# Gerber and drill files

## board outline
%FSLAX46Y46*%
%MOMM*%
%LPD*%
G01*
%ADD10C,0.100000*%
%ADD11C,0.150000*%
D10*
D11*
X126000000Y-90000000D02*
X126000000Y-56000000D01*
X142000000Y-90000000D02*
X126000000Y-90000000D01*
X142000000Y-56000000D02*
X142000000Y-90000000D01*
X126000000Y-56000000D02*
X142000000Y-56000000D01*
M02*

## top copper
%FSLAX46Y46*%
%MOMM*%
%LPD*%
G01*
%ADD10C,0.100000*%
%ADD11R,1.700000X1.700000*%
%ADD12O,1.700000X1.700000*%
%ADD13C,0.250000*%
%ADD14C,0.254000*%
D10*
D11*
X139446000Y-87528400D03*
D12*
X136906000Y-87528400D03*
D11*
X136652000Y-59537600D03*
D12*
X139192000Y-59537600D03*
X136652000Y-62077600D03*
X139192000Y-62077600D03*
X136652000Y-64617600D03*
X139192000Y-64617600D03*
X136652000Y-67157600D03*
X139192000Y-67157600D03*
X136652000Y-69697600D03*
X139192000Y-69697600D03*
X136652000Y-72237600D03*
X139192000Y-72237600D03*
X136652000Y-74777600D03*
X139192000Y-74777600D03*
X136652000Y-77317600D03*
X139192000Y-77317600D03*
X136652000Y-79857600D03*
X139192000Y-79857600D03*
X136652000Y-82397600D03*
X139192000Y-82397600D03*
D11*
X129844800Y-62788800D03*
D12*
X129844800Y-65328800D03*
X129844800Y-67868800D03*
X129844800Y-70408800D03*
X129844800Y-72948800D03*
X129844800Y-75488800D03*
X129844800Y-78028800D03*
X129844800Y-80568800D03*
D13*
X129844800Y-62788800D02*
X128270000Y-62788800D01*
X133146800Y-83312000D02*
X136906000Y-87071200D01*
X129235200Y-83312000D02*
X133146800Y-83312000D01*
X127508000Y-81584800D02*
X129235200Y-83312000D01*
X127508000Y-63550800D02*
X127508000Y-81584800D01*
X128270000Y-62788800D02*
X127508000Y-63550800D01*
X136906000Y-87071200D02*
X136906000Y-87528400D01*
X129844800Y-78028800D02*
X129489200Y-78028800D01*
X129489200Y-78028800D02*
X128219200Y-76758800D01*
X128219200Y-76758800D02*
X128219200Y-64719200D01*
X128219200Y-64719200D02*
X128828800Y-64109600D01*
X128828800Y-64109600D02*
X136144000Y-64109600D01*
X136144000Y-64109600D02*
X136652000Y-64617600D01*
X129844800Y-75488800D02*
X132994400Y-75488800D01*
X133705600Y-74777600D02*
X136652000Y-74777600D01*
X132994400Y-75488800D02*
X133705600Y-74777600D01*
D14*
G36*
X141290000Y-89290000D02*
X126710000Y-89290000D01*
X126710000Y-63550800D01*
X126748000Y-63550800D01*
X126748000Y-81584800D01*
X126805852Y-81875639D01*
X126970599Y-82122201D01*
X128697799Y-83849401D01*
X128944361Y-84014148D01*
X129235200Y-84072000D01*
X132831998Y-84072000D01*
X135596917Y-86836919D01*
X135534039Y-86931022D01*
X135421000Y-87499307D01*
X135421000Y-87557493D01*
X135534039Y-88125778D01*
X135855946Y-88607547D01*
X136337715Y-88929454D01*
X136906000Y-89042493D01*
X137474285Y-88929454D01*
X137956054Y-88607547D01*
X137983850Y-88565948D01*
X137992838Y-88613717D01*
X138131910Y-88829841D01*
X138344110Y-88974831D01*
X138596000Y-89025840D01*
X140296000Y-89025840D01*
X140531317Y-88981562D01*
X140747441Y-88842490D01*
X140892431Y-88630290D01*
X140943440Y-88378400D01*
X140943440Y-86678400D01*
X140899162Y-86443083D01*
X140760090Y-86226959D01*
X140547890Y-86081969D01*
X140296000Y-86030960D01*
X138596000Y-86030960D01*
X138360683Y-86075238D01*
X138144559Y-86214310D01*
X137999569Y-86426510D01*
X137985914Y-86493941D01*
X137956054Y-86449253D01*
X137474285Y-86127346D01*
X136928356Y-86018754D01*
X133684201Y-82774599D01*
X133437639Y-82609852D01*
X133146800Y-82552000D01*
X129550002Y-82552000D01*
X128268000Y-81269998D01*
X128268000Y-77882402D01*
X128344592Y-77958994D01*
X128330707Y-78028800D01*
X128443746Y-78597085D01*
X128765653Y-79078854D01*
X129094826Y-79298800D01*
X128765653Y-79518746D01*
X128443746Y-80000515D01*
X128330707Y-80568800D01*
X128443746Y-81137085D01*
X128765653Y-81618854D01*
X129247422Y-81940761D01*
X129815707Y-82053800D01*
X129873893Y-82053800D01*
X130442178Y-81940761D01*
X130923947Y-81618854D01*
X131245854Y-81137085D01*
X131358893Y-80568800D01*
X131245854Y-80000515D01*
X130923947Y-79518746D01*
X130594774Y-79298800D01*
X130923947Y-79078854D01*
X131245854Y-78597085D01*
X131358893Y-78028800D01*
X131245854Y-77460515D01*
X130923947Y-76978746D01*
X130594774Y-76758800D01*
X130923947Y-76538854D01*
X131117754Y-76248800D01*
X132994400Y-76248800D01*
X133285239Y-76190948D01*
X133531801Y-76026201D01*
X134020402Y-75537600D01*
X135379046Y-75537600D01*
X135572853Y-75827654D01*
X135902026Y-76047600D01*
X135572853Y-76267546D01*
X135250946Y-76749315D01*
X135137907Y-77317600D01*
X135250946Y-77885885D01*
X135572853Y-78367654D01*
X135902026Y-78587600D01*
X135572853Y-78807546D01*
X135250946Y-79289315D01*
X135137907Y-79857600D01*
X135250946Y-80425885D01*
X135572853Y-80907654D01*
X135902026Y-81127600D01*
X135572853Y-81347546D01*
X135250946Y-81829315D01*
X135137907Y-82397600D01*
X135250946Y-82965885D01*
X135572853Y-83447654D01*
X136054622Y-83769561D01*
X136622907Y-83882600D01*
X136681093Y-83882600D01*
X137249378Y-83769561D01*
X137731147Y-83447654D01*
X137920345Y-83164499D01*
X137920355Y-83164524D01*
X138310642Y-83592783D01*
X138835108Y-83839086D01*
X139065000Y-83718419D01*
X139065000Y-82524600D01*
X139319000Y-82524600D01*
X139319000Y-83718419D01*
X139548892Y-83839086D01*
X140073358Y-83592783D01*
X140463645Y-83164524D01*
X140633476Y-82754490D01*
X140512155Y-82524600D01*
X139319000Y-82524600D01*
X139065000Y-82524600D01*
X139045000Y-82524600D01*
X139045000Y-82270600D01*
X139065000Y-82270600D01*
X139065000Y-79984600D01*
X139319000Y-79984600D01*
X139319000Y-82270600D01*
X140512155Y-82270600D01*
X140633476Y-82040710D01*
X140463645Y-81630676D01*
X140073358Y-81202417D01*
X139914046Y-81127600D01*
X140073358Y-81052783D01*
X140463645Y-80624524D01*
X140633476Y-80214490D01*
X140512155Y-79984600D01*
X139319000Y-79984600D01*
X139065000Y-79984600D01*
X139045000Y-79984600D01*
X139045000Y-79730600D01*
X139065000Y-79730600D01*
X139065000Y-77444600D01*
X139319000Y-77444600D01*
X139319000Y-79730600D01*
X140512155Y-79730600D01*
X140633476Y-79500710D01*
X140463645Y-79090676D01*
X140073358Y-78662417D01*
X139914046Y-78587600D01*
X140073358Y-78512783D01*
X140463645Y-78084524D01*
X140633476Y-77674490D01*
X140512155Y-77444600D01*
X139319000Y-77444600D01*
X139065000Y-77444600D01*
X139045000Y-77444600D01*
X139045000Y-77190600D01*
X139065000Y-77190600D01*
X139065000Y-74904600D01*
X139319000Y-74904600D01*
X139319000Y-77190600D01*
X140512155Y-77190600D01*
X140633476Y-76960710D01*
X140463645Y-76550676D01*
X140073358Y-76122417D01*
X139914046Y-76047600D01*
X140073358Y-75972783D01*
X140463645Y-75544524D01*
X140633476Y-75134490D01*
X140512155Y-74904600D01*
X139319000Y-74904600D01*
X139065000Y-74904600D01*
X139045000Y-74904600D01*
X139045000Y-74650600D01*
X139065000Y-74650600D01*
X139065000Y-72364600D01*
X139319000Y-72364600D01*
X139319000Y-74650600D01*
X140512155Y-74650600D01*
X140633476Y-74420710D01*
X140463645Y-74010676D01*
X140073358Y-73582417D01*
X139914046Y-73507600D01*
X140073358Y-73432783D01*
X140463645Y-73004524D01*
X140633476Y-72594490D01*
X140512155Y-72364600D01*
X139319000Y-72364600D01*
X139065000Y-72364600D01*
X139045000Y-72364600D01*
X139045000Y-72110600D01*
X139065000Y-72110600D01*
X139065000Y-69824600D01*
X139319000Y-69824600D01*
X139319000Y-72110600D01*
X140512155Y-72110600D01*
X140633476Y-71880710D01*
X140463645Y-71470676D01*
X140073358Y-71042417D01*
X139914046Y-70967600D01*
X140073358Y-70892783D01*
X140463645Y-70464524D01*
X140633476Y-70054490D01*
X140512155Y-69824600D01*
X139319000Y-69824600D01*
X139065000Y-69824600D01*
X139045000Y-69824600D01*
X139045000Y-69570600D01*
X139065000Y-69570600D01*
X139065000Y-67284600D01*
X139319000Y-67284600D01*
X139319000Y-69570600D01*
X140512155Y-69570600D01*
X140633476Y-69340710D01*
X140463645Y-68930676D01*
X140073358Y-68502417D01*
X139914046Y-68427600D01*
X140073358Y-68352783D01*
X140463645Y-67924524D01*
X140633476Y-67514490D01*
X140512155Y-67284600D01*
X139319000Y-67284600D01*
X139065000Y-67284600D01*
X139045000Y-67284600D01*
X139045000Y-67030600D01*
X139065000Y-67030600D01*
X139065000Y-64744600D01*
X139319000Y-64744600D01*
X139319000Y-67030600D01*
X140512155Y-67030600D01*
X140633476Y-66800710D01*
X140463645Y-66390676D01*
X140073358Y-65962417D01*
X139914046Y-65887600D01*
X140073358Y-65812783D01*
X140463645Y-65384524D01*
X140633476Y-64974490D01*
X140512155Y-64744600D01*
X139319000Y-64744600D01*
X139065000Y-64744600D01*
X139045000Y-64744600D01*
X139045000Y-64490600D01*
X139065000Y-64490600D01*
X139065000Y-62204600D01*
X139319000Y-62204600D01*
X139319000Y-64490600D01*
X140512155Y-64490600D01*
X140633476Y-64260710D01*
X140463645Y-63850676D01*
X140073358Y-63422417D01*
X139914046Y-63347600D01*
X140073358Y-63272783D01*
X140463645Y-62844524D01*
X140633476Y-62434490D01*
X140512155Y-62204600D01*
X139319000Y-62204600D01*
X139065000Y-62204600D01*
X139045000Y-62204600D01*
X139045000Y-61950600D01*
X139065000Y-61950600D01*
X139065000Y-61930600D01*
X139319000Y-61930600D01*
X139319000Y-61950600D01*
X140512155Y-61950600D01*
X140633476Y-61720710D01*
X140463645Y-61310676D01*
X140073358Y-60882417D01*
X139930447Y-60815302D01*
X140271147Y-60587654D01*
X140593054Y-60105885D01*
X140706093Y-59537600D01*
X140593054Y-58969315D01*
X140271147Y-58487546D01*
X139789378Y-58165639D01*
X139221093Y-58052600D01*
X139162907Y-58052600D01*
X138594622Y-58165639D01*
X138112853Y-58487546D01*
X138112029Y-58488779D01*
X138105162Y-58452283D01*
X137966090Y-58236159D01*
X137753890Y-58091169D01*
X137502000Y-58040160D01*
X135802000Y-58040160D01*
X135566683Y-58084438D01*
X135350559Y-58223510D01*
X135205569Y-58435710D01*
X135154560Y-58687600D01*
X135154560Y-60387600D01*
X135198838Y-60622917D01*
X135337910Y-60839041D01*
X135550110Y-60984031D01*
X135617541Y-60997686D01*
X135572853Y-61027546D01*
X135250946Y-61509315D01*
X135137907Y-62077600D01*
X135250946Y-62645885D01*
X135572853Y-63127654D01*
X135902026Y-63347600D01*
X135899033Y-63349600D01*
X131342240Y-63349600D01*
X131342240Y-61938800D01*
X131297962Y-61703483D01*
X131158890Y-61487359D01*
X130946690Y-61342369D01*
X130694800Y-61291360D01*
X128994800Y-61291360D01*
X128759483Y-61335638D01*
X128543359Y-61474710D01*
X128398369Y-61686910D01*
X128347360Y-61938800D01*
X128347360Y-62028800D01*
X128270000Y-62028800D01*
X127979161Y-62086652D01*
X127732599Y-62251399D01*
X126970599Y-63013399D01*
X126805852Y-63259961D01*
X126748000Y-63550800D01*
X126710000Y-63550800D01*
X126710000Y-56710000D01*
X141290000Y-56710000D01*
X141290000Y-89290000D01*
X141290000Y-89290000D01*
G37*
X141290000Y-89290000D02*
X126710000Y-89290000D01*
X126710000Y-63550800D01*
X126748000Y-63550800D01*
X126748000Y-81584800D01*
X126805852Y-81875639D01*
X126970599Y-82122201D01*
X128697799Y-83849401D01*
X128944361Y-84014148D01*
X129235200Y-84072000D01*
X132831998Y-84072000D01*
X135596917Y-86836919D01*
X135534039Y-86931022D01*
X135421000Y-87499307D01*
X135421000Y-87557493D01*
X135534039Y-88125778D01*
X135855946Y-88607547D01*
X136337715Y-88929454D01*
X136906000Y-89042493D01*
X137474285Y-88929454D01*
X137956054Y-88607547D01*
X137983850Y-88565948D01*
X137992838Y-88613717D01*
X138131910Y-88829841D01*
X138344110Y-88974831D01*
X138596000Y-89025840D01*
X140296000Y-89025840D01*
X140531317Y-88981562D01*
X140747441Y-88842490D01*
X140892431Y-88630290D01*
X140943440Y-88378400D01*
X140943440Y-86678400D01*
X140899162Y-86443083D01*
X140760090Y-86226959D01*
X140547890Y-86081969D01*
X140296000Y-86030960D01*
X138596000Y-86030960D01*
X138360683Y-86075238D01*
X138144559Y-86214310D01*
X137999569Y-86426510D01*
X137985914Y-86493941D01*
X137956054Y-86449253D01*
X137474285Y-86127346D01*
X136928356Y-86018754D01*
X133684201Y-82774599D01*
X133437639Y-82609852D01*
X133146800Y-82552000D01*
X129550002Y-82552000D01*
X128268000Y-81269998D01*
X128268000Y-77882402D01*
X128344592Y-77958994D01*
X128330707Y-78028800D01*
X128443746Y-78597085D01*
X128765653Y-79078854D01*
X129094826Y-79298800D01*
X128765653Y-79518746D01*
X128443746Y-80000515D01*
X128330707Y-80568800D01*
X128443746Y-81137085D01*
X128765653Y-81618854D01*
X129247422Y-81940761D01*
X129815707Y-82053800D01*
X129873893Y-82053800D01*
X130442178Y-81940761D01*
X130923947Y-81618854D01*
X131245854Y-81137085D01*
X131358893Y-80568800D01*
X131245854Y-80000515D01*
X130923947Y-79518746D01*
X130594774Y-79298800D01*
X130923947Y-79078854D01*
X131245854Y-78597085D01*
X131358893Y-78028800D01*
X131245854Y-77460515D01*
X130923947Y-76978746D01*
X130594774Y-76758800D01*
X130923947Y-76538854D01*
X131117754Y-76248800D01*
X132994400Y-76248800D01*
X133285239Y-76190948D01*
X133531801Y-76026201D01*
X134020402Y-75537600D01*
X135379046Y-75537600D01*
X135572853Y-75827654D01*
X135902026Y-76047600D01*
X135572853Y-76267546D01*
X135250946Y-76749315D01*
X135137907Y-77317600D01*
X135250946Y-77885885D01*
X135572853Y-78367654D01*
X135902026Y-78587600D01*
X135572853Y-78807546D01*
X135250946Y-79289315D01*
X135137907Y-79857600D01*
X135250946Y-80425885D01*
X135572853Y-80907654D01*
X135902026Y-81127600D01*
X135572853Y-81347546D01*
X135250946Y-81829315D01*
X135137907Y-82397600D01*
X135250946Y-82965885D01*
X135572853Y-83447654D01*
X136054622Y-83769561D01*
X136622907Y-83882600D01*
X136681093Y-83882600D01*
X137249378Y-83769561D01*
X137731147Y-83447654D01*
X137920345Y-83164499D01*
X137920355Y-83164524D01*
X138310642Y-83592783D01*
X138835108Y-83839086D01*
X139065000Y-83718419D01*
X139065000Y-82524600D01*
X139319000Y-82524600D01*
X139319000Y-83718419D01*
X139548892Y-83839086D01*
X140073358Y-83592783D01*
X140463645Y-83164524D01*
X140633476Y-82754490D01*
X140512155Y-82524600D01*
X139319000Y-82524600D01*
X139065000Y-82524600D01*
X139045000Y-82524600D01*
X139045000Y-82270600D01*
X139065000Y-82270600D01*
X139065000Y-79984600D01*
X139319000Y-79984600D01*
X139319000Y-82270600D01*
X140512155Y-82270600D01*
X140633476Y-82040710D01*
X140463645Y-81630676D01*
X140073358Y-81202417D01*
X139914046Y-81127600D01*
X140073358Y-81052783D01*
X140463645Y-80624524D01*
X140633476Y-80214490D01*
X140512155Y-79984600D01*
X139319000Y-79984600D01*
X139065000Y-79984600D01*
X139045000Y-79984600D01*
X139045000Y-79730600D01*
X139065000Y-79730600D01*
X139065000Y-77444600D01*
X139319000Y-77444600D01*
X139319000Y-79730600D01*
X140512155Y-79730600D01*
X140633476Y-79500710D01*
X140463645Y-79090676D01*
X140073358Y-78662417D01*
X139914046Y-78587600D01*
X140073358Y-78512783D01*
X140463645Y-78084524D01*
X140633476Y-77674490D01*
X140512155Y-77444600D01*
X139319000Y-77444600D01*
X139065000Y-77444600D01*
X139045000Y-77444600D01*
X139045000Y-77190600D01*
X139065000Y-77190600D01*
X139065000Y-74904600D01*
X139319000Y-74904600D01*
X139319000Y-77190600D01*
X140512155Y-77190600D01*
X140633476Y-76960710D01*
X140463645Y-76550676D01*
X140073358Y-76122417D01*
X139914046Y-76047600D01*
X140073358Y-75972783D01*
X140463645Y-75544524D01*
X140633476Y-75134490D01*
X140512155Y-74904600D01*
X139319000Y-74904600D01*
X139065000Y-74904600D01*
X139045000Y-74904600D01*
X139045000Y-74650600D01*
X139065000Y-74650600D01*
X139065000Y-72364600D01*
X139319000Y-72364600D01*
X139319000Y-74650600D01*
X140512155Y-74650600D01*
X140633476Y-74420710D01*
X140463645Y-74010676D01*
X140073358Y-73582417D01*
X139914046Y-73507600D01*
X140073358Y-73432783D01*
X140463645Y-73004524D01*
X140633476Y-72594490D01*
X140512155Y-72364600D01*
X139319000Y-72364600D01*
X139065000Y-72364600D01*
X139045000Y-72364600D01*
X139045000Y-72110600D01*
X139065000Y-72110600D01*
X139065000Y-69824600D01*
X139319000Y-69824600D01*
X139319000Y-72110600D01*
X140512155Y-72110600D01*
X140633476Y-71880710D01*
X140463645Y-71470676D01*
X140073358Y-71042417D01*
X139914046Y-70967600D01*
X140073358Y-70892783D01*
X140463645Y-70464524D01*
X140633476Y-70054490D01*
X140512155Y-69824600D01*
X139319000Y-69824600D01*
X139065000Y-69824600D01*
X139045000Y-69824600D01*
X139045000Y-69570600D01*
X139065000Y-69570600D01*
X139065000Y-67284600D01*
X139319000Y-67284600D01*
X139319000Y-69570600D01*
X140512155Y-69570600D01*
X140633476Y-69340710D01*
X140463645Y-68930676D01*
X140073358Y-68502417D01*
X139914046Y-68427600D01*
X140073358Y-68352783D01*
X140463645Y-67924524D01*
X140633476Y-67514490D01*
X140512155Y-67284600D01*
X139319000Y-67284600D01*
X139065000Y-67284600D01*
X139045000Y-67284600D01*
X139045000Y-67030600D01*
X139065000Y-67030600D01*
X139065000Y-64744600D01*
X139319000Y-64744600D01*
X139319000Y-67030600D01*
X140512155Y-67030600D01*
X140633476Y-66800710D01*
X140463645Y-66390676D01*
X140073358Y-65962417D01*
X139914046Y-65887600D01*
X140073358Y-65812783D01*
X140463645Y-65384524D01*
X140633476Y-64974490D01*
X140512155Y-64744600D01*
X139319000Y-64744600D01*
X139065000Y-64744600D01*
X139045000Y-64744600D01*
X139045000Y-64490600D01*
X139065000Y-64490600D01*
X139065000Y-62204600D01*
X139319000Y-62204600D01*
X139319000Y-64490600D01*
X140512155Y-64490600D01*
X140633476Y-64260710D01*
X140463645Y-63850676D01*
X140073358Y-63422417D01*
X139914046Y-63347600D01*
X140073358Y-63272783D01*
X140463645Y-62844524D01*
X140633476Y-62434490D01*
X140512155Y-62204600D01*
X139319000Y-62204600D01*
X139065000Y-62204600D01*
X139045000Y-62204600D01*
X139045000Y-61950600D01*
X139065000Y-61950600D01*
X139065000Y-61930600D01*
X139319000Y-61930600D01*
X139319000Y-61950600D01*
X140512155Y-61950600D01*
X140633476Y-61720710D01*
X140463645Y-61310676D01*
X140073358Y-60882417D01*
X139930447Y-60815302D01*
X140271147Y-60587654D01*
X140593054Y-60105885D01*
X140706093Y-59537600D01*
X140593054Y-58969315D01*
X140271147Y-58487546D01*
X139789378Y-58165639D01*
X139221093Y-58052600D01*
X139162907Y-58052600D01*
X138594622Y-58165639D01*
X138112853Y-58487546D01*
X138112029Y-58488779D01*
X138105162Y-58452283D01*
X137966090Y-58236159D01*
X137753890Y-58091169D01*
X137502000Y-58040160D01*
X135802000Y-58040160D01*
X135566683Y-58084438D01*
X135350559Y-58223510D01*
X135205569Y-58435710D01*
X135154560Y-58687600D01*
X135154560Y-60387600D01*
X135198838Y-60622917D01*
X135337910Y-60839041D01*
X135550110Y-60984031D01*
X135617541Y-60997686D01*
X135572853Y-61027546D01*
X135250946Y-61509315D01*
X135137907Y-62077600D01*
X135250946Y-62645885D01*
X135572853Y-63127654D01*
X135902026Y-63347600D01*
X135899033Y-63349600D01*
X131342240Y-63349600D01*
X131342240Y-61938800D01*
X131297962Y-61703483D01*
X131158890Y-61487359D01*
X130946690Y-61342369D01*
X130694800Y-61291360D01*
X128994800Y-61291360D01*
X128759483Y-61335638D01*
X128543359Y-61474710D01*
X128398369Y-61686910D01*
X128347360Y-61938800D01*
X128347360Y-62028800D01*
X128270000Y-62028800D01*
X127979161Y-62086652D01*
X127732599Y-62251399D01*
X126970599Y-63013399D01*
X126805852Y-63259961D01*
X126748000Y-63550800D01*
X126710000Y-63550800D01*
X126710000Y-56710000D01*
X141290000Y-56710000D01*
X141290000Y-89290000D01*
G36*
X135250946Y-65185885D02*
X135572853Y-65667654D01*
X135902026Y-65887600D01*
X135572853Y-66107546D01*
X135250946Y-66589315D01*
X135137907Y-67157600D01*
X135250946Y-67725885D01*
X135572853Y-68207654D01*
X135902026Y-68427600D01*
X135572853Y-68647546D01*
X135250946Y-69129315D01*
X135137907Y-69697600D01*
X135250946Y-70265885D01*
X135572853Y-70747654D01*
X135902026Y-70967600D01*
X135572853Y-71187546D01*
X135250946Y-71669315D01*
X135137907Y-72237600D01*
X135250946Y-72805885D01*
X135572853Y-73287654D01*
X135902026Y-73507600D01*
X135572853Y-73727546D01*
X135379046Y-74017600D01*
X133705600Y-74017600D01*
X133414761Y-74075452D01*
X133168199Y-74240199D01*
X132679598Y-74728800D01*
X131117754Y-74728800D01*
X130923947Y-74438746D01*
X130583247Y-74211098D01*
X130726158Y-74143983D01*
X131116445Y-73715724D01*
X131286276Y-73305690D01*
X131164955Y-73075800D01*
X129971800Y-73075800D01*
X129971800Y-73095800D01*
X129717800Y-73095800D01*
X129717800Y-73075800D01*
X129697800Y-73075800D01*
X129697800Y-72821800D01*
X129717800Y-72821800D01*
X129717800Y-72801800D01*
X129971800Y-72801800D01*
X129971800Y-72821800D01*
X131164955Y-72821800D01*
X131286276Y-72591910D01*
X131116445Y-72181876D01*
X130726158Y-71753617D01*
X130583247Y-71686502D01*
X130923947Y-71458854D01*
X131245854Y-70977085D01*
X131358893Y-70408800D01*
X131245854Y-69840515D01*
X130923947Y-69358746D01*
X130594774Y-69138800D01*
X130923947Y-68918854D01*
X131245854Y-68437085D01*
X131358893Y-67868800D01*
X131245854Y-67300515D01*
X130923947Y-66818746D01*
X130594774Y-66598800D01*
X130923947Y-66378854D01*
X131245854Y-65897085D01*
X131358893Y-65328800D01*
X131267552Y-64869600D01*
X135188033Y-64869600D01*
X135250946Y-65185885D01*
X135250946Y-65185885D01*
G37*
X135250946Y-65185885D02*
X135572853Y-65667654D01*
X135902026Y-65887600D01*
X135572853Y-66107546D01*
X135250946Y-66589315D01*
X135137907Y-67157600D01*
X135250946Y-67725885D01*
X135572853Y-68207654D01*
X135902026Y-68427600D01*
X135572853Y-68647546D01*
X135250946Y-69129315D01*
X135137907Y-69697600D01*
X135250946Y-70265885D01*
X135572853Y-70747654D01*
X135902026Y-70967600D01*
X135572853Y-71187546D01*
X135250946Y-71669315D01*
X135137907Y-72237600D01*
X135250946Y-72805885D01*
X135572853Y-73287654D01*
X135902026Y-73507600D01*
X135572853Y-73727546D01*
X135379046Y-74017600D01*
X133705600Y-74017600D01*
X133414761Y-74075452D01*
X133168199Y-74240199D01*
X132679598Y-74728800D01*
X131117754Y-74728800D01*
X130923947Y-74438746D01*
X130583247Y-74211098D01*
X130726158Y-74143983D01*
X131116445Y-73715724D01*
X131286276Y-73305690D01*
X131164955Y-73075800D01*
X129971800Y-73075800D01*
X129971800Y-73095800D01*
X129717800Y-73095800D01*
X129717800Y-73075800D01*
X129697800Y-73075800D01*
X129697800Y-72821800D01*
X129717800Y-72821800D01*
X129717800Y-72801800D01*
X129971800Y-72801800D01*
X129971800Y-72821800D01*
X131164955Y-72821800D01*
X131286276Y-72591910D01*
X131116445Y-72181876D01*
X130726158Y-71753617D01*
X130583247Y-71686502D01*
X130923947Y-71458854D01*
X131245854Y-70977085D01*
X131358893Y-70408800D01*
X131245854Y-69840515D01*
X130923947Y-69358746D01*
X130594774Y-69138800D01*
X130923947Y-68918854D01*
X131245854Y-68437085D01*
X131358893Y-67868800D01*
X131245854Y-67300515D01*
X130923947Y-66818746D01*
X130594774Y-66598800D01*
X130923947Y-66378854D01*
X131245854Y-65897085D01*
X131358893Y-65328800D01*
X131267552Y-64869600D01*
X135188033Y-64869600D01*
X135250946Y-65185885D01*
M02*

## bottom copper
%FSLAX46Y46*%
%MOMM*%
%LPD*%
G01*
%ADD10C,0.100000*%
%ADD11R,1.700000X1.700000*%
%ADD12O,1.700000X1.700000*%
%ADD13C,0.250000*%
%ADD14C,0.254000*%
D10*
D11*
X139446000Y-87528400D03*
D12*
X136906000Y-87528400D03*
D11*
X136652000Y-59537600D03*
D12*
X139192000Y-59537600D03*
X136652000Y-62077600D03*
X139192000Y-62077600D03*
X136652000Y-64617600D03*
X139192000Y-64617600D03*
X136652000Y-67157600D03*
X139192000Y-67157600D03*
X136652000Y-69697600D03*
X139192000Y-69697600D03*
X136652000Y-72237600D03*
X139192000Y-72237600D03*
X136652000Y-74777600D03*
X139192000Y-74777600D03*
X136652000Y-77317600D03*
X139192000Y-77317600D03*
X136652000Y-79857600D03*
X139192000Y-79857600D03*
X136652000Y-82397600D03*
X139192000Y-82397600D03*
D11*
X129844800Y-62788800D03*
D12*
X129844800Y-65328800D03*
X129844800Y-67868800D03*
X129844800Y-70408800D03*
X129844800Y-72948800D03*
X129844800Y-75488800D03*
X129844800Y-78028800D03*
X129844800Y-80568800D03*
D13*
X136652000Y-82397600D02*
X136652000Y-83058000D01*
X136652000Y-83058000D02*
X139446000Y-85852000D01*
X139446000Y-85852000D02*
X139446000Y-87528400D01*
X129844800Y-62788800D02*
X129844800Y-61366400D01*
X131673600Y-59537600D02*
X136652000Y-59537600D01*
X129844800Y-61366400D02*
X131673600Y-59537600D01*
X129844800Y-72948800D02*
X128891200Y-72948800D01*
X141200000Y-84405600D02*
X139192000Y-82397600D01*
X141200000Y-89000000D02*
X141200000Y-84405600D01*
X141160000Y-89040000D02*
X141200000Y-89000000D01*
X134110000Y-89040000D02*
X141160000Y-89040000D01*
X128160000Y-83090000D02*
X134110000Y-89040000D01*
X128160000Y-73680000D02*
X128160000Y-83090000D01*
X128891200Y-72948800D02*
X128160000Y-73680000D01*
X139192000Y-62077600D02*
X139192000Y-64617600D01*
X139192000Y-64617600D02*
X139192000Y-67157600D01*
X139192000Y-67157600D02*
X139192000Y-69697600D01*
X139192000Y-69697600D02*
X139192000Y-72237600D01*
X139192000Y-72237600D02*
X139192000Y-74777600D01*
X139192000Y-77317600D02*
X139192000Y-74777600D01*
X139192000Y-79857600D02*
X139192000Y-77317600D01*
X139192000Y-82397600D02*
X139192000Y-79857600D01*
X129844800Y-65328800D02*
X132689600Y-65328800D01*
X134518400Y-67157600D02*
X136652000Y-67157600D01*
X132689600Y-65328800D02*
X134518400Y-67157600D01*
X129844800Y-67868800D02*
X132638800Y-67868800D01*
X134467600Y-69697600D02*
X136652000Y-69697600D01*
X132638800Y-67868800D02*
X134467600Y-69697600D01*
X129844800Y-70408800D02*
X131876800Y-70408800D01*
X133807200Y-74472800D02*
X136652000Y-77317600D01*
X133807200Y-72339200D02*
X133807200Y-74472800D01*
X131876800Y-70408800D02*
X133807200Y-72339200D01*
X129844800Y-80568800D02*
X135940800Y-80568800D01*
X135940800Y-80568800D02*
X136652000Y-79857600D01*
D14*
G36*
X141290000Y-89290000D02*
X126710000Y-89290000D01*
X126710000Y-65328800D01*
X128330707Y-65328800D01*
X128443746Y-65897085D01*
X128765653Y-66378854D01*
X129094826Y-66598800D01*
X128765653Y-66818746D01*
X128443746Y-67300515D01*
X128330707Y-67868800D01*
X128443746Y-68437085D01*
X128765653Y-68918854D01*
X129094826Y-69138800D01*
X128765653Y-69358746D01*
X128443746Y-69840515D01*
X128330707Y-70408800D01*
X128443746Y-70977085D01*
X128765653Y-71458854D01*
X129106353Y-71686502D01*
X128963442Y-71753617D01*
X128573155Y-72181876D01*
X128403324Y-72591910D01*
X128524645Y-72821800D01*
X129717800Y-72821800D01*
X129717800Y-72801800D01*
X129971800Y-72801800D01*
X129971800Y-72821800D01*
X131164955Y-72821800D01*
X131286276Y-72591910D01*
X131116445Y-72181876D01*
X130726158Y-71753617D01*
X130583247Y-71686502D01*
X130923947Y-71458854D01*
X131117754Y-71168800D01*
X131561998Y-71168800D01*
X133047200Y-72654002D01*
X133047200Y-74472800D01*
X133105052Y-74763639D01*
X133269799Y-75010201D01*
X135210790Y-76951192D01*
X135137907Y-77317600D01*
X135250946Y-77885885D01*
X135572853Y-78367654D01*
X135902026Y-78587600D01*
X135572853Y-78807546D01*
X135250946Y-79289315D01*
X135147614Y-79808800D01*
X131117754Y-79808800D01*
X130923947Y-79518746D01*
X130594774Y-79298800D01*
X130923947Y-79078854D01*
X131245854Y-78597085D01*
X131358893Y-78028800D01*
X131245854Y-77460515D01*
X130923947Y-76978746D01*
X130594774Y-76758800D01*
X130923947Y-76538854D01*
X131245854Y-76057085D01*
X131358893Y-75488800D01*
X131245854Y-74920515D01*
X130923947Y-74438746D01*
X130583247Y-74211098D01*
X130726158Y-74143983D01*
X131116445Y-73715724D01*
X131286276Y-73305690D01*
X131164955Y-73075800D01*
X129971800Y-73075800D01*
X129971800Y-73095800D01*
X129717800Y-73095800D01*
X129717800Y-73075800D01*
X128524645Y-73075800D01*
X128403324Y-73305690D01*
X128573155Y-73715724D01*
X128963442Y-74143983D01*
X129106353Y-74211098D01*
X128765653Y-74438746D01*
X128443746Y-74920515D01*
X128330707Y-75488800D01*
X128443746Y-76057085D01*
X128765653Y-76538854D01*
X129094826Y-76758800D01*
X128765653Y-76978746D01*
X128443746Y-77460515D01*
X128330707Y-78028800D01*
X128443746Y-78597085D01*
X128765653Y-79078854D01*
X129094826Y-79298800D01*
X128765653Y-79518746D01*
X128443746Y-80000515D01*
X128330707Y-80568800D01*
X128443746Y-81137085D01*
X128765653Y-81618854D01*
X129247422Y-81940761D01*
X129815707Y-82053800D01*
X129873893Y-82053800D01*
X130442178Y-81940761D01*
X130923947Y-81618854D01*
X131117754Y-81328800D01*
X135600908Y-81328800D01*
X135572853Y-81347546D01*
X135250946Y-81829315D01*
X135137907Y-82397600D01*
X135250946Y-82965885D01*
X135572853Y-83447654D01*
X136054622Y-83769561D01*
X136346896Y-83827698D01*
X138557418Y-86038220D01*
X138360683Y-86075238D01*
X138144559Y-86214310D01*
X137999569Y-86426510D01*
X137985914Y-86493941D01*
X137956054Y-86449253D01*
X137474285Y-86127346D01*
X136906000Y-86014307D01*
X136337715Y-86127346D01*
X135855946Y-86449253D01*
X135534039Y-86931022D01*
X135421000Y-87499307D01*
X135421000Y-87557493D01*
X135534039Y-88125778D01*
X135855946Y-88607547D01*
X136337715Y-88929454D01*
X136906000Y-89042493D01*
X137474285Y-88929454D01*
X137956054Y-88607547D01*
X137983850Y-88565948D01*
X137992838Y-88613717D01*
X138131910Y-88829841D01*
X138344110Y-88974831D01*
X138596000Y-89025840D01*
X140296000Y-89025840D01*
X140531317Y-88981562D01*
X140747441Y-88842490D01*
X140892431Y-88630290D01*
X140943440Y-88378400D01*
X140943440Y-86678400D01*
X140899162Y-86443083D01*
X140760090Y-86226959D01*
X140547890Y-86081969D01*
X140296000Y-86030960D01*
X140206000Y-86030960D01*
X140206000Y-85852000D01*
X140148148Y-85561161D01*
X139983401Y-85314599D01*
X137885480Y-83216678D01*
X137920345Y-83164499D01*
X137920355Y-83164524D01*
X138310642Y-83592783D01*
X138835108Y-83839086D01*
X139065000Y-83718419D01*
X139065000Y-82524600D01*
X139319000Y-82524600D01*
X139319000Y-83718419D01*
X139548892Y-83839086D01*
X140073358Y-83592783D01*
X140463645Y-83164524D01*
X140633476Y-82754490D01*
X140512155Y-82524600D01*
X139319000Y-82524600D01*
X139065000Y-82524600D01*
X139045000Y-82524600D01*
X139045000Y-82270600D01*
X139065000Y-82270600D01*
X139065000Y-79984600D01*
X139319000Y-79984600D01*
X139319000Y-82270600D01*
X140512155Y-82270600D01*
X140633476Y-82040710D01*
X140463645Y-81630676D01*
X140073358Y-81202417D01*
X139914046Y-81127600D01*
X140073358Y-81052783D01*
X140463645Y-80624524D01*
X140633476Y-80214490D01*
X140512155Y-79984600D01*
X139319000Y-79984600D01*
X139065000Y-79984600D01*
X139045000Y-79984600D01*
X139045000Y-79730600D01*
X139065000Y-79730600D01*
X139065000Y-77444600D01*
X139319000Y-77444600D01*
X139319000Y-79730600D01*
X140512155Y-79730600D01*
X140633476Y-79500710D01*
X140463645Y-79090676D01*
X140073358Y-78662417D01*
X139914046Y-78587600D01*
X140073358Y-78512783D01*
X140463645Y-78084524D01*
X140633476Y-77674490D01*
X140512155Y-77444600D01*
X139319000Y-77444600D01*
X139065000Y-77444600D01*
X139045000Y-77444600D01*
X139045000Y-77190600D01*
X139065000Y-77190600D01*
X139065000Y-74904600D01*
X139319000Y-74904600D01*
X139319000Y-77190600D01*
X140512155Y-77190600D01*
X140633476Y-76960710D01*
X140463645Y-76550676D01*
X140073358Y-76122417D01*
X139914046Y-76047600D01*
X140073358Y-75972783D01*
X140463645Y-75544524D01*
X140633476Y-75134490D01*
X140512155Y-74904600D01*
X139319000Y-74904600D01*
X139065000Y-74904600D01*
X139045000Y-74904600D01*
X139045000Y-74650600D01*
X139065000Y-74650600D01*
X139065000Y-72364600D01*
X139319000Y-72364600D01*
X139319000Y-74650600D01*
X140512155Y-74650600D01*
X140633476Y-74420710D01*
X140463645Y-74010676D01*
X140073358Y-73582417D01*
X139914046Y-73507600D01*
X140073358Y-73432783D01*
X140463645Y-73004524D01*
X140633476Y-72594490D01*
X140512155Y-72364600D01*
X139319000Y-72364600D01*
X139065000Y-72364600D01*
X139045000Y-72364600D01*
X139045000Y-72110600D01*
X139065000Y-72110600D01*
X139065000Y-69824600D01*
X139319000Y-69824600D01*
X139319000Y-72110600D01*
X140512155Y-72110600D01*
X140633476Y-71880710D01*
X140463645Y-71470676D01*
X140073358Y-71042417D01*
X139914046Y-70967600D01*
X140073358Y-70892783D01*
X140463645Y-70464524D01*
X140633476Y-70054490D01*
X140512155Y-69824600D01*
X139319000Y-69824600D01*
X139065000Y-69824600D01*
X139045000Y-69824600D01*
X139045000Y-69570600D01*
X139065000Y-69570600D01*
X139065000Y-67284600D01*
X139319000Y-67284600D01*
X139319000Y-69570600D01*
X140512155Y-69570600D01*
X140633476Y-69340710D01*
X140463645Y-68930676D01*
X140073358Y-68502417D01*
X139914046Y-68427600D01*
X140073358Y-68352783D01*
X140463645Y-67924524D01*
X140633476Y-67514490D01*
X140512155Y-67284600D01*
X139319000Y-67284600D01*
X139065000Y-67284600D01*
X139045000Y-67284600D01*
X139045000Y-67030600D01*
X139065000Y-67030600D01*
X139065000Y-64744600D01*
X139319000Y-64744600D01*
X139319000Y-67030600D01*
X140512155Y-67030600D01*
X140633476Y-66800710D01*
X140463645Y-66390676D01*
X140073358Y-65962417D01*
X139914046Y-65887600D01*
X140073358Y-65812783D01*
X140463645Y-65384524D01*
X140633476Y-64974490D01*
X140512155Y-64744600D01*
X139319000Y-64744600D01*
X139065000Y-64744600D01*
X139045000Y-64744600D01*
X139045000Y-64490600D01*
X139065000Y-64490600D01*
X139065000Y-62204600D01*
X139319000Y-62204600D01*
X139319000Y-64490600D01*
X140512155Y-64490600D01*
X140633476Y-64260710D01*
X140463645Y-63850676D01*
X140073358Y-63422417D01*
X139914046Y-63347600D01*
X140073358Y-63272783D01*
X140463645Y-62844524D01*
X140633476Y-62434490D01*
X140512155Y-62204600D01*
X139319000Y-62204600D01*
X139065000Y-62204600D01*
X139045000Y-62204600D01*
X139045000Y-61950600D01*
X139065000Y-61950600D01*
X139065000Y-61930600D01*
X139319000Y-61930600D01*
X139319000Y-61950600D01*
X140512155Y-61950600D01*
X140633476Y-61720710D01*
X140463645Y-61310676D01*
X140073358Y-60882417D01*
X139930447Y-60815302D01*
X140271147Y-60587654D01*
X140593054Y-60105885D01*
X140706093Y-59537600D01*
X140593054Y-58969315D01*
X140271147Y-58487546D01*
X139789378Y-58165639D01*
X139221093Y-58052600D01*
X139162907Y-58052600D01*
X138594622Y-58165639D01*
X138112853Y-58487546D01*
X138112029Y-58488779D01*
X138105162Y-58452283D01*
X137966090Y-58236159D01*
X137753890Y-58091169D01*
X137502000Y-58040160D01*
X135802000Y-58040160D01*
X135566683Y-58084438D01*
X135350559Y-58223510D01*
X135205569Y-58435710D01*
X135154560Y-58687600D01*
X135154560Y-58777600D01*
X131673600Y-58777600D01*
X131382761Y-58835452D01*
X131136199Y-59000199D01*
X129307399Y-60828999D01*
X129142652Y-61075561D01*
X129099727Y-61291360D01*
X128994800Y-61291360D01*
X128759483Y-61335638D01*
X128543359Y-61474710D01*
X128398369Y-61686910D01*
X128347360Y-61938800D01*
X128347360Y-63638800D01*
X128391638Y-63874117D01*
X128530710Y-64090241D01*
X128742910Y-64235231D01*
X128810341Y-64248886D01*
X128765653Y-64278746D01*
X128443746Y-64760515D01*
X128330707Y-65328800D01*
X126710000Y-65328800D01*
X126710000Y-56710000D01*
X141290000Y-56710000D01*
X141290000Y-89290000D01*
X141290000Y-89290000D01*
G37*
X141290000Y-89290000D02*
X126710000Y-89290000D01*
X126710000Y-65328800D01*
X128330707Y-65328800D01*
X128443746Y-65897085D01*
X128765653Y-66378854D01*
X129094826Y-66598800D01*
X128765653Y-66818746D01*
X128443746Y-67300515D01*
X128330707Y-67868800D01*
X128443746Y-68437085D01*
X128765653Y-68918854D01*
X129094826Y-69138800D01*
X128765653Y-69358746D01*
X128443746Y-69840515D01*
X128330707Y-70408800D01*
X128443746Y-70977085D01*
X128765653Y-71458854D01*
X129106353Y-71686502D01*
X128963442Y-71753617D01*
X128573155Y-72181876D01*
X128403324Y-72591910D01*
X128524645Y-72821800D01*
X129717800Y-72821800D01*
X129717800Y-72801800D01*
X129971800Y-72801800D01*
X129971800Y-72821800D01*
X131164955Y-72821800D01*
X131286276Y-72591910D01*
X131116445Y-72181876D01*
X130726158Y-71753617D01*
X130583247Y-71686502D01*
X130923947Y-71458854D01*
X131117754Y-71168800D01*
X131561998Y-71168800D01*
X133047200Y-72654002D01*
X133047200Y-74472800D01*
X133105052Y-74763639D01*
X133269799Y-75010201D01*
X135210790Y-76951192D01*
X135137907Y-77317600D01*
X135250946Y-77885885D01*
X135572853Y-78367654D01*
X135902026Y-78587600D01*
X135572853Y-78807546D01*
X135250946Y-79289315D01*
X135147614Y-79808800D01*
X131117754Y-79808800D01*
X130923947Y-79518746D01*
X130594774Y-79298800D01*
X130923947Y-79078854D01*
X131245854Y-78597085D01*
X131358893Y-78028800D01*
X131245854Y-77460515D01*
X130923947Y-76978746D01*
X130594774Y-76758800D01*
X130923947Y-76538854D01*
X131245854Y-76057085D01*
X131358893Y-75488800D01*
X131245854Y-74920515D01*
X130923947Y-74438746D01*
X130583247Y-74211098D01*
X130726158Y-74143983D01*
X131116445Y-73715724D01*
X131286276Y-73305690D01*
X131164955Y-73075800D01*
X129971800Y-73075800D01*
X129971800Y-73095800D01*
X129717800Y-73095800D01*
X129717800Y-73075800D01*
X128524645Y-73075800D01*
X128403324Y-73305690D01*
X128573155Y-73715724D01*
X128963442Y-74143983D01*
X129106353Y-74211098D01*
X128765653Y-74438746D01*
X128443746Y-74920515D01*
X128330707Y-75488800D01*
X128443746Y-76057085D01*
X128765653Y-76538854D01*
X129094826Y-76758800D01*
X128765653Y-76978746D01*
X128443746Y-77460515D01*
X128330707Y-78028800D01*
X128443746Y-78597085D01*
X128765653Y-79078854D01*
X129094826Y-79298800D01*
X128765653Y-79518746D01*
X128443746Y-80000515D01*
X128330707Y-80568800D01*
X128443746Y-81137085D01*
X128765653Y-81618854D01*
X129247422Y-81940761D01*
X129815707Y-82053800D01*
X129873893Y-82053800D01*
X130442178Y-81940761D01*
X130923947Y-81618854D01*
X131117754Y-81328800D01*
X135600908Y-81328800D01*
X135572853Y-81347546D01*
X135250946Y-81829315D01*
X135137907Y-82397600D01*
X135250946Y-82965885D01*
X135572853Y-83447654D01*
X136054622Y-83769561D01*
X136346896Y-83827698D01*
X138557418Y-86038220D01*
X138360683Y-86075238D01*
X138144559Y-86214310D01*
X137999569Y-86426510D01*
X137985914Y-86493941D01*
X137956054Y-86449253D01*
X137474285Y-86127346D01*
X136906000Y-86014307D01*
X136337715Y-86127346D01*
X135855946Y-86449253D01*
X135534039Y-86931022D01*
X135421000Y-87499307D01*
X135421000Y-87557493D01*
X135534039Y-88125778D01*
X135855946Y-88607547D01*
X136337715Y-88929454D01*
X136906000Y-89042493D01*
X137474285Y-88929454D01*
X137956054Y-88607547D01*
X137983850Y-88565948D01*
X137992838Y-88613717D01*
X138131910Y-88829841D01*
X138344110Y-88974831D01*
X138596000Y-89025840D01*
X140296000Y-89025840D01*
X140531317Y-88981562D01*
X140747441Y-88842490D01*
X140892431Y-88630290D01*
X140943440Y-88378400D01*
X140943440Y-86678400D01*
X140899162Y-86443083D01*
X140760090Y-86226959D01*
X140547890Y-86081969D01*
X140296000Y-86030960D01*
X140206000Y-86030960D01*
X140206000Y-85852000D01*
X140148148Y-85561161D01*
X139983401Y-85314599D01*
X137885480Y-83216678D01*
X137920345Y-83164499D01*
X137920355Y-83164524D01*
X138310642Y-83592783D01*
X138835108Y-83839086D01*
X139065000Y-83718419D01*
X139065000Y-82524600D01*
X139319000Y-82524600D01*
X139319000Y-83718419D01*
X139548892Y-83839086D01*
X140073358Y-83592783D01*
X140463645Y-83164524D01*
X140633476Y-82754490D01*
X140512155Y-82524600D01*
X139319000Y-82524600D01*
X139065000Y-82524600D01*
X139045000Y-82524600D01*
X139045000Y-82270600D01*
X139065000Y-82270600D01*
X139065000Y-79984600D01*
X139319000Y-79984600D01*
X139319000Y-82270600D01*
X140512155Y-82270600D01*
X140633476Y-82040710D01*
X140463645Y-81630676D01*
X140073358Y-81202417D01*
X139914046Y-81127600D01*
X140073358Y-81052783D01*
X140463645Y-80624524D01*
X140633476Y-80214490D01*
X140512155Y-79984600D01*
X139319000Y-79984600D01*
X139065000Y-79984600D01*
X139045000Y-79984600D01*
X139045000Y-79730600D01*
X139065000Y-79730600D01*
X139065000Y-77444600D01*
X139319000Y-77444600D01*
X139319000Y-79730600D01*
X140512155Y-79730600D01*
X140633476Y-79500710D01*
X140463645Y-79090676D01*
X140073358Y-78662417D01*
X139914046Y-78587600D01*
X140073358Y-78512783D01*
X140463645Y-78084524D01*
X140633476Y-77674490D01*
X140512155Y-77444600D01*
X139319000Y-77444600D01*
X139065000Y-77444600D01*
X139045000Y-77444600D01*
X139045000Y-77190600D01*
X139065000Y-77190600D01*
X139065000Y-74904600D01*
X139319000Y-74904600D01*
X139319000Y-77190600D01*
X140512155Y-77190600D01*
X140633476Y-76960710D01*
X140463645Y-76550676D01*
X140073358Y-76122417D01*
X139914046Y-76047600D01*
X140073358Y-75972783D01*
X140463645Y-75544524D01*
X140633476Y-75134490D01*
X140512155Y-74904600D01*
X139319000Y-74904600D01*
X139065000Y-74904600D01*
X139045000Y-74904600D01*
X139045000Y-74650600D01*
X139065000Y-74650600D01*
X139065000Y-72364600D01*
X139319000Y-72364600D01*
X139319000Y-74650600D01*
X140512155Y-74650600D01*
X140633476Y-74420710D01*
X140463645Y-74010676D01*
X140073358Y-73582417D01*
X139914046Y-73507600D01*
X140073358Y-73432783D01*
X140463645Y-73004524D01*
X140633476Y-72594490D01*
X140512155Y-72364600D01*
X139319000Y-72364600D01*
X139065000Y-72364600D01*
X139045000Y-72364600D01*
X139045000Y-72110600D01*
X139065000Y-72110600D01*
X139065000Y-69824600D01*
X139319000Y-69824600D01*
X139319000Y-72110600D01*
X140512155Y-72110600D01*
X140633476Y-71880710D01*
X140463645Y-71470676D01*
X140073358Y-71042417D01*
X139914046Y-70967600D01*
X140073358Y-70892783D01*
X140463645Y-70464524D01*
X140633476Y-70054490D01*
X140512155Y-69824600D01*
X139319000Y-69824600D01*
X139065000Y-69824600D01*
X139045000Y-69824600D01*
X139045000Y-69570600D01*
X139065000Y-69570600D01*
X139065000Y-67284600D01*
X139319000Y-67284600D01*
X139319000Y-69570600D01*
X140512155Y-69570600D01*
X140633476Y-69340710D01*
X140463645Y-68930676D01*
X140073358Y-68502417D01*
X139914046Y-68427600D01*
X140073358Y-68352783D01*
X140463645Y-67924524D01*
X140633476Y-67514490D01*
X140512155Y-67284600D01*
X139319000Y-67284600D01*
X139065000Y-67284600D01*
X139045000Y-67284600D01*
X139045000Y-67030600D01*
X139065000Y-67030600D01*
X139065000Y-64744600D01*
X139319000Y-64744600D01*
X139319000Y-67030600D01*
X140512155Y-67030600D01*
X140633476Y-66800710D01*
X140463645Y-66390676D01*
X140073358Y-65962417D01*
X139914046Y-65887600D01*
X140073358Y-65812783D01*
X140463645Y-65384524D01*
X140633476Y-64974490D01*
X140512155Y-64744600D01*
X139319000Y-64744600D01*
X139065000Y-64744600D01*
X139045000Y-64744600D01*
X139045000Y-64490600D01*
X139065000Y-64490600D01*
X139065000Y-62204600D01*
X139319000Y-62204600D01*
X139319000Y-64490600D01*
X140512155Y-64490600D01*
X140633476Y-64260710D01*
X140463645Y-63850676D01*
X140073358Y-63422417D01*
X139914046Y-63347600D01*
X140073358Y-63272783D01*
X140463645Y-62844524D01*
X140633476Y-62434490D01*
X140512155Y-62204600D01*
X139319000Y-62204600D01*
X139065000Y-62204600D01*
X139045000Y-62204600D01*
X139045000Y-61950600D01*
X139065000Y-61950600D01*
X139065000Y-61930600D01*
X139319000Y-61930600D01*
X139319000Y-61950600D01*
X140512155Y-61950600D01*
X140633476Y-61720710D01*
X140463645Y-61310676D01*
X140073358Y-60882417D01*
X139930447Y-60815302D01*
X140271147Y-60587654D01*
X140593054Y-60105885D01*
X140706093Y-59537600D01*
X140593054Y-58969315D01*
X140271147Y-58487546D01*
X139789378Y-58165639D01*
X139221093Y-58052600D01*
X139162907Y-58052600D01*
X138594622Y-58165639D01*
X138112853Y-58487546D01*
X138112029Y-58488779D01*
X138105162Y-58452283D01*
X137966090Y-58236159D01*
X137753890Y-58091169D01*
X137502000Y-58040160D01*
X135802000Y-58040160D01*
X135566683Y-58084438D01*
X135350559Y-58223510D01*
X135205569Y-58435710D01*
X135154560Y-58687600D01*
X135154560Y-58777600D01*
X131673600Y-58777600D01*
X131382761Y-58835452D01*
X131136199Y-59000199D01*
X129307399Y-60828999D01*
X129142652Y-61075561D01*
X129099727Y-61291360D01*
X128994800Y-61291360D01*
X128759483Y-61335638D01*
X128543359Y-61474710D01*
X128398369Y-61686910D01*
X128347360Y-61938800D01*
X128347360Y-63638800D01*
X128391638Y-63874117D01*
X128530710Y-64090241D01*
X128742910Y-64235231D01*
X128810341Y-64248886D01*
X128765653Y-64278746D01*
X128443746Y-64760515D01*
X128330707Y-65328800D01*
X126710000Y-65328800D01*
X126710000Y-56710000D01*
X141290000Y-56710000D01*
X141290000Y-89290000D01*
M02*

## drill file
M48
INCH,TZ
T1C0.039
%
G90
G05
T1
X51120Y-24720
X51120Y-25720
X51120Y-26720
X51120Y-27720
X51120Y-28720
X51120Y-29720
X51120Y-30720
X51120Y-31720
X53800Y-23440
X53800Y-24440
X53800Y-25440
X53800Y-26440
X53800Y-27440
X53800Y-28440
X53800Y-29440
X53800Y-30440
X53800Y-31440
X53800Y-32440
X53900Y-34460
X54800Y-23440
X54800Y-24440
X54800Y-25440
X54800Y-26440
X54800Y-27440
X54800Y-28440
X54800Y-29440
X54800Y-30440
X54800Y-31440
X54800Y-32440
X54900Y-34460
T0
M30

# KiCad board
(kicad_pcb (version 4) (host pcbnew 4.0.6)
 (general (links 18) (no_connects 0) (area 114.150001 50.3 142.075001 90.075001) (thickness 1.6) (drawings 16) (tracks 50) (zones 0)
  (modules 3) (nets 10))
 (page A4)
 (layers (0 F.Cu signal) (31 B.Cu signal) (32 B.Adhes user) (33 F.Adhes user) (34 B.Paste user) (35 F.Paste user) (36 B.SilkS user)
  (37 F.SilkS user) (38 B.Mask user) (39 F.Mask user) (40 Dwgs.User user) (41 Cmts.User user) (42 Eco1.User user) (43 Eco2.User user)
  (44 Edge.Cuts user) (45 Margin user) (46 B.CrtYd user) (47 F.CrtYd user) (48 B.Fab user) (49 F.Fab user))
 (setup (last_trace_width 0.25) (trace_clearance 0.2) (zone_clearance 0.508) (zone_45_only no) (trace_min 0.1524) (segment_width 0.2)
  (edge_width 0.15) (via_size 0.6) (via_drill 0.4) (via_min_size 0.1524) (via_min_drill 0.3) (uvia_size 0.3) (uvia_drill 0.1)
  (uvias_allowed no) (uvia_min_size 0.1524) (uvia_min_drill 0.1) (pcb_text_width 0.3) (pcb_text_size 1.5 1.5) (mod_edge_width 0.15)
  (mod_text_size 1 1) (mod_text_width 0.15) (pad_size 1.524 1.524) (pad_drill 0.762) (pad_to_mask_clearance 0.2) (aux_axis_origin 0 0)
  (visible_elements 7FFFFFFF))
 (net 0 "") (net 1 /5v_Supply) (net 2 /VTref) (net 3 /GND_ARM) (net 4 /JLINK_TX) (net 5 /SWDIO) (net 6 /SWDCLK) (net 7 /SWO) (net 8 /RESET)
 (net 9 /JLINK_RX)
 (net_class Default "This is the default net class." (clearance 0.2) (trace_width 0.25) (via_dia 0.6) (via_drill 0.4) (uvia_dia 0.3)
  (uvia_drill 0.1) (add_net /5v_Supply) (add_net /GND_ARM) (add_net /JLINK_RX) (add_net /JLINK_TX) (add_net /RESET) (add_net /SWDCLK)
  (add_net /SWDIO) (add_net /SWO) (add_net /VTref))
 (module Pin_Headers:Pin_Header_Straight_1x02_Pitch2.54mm (layer F.Cu) (at 139.446 87.5284 270)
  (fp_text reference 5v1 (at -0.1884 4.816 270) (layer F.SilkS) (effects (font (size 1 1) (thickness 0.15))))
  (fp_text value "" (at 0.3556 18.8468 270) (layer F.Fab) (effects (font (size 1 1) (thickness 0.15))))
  (pad 1 thru_hole rect (at 0 0 270) (size 1.7 1.7) (drill 1) (layers *.Cu *.Mask) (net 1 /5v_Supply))
  (pad 2 thru_hole oval (at 0 2.54 270) (size 1.7 1.7) (drill 1) (layers *.Cu *.Mask) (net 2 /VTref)))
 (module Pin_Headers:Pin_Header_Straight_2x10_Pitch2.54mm (layer F.Cu) (at 136.652 59.5376)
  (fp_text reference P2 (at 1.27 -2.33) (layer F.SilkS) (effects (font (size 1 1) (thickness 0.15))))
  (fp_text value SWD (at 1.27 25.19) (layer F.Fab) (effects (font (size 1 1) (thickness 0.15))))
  (pad 1 thru_hole rect (at 0 0) (size 1.7 1.7) (drill 1) (layers *.Cu *.Mask) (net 2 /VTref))
  (pad 2 thru_hole oval (at 2.54 0) (size 1.7 1.7) (drill 1) (layers *.Cu *.Mask))
  (pad 3 thru_hole oval (at 0 2.54) (size 1.7 1.7) (drill 1) (layers *.Cu *.Mask))
  (pad 4 thru_hole oval (at 2.54 2.54) (size 1.7 1.7) (drill 1) (layers *.Cu *.Mask) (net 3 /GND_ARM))
  (pad 5 thru_hole oval (at 0 5.08) (size 1.7 1.7) (drill 1) (layers *.Cu *.Mask) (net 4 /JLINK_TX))
  (pad 6 thru_hole oval (at 2.54 5.08) (size 1.7 1.7) (drill 1) (layers *.Cu *.Mask) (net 3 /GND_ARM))
  (pad 7 thru_hole oval (at 0 7.62) (size 1.7 1.7) (drill 1) (layers *.Cu *.Mask) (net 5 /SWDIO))
  (pad 8 thru_hole oval (at 2.54 7.62) (size 1.7 1.7) (drill 1) (layers *.Cu *.Mask) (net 3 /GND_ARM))
  (pad 9 thru_hole oval (at 0 10.16) (size 1.7 1.7) (drill 1) (layers *.Cu *.Mask) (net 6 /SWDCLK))
  (pad 10 thru_hole oval (at 2.54 10.16) (size 1.7 1.7) (drill 1) (layers *.Cu *.Mask) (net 3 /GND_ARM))
  (pad 11 thru_hole oval (at 0 12.7) (size 1.7 1.7) (drill 1) (layers *.Cu *.Mask))
  (pad 12 thru_hole oval (at 2.54 12.7) (size 1.7 1.7) (drill 1) (layers *.Cu *.Mask) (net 3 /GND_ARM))
  (pad 13 thru_hole oval (at 0 15.24) (size 1.7 1.7) (drill 1) (layers *.Cu *.Mask) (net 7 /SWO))
  (pad 14 thru_hole oval (at 2.54 15.24) (size 1.7 1.7) (drill 1) (layers *.Cu *.Mask) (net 3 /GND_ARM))
  (pad 15 thru_hole oval (at 0 17.78) (size 1.7 1.7) (drill 1) (layers *.Cu *.Mask) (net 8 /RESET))
  (pad 16 thru_hole oval (at 2.54 17.78) (size 1.7 1.7) (drill 1) (layers *.Cu *.Mask) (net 3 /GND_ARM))
  (pad 17 thru_hole oval (at 0 20.32) (size 1.7 1.7) (drill 1) (layers *.Cu *.Mask) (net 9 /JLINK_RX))
  (pad 18 thru_hole oval (at 2.54 20.32) (size 1.7 1.7) (drill 1) (layers *.Cu *.Mask) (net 3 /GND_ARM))
  (pad 19 thru_hole oval (at 0 22.86) (size 1.7 1.7) (drill 1) (layers *.Cu *.Mask) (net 1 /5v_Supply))
  (pad 20 thru_hole oval (at 2.54 22.86) (size 1.7 1.7) (drill 1) (layers *.Cu *.Mask) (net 3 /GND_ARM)))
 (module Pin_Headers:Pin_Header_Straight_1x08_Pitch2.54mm (layer F.Cu) (at 129.8448 62.7888)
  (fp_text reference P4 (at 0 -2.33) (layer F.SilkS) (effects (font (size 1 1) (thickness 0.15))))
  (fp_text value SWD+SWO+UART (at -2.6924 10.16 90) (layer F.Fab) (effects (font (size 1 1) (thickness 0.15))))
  (pad 1 thru_hole rect (at 0 0) (size 1.7 1.7) (drill 1) (layers *.Cu *.Mask) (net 2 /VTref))
  (pad 2 thru_hole oval (at 0 2.54) (size 1.7 1.7) (drill 1) (layers *.Cu *.Mask) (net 5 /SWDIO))
  (pad 3 thru_hole oval (at 0 5.08) (size 1.7 1.7) (drill 1) (layers *.Cu *.Mask) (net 6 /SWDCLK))
  (pad 4 thru_hole oval (at 0 7.62) (size 1.7 1.7) (drill 1) (layers *.Cu *.Mask) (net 8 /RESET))
  (pad 5 thru_hole oval (at 0 10.16) (size 1.7 1.7) (drill 1) (layers *.Cu *.Mask) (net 3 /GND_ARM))
  (pad 6 thru_hole oval (at 0 12.7) (size 1.7 1.7) (drill 1) (layers *.Cu *.Mask) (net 7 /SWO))
  (pad 7 thru_hole oval (at 0 15.24) (size 1.7 1.7) (drill 1) (layers *.Cu *.Mask) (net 4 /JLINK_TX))
  (pad 8 thru_hole oval (at 0 17.78) (size 1.7 1.7) (drill 1) (layers *.Cu *.Mask) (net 9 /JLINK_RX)))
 (gr_line (start 126 90) (end 126 56) (angle 90) (layer Edge.Cuts) (width 0.15))
 (gr_line (start 142 90) (end 126 90) (angle 90) (layer Edge.Cuts) (width 0.15))
 (gr_line (start 142 56) (end 142 90) (angle 90) (layer Edge.Cuts) (width 0.15))
 (gr_line (start 126 56) (end 142 56) (angle 90) (layer Edge.Cuts) (width 0.15))
 (segment (start 136.652 82.3976) (end 136.652 83.058) (width 0.25) (layer B.Cu) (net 1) (status C00000))
 (segment (start 136.652 83.058) (end 139.446 85.852) (width 0.25) (layer B.Cu) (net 1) (status 400000))
 (segment (start 139.446 85.852) (end 139.446 87.5284) (width 0.25) (layer B.Cu) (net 1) (status 800000))
 (segment (start 129.8448 62.7888) (end 128.27 62.7888) (width 0.25) (layer F.Cu) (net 2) (status 400000))
 (segment (start 133.1468 83.312) (end 136.906 87.0712) (width 0.25) (layer F.Cu) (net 2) (status 800000))
 (segment (start 129.2352 83.312) (end 133.1468 83.312) (width 0.25) (layer F.Cu) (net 2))
 (segment (start 127.508 81.5848) (end 129.2352 83.312) (width 0.25) (layer F.Cu) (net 2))
 (segment (start 127.508 63.5508) (end 127.508 81.5848) (width 0.25) (layer F.Cu) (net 2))
 (segment (start 128.27 62.7888) (end 127.508 63.5508) (width 0.25) (layer F.Cu) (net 2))
 (segment (start 136.906 87.0712) (end 136.906 87.5284) (width 0.25) (layer F.Cu) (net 2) (status C00000))
 (segment (start 129.8448 62.7888) (end 129.8448 61.3664) (width 0.25) (layer B.Cu) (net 2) (status 400000))
 (segment (start 131.6736 59.5376) (end 136.652 59.5376) (width 0.25) (layer B.Cu) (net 2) (status 800000))
 (segment (start 129.8448 61.3664) (end 131.6736 59.5376) (width 0.25) (layer B.Cu) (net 2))
 (segment (start 129.8448 72.9488) (end 128.8912 72.9488) (width 0.25) (layer B.Cu) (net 3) (status 400000))
 (segment (start 141.2 84.4056) (end 139.192 82.3976) (width 0.25) (layer B.Cu) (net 3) (status 800000))
 (segment (start 141.2 89) (end 141.2 84.4056) (width 0.25) (layer B.Cu) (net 3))
 (segment (start 141.16 89.04) (end 141.2 89) (width 0.25) (layer B.Cu) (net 3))
 (segment (start 134.11 89.04) (end 141.16 89.04) (width 0.25) (layer B.Cu) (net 3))
 (segment (start 128.16 83.09) (end 134.11 89.04) (width 0.25) (layer B.Cu) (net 3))
 (segment (start 128.16 73.68) (end 128.16 83.09) (width 0.25) (layer B.Cu) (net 3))
 (segment (start 128.8912 72.9488) (end 128.16 73.68) (width 0.25) (layer B.Cu) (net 3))
 (segment (start 139.192 62.0776) (end 139.192 64.6176) (width 0.25) (layer B.Cu) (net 3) (status C00000))
 (segment (start 139.192 64.6176) (end 139.192 67.1576) (width 0.25) (layer B.Cu) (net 3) (status C00000))
 (segment (start 139.192 67.1576) (end 139.192 69.6976) (width 0.25) (layer B.Cu) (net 3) (status C00000))
 (segment (start 139.192 69.6976) (end 139.192 72.2376) (width 0.25) (layer B.Cu) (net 3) (status C00000))
 (segment (start 139.192 72.2376) (end 139.192 74.7776) (width 0.25) (layer B.Cu) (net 3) (status C00000))
 (segment (start 139.192 77.3176) (end 139.192 74.7776) (width 0.25) (layer B.Cu) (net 3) (status C00000))
 (segment (start 139.192 79.8576) (end 139.192 77.3176) (width 0.25) (layer B.Cu) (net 3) (status C00000))
 (segment (start 139.192 82.3976) (end 139.192 79.8576) (width 0.25) (layer B.Cu) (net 3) (status C00000))
 (segment (start 129.8448 78.0288) (end 129.4892 78.0288) (width 0.25) (layer F.Cu) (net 4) (status C00000))
 (segment (start 129.4892 78.0288) (end 128.2192 76.7588) (width 0.25) (layer F.Cu) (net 4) (status 400000))
 (segment (start 128.2192 76.7588) (end 128.2192 64.7192) (width 0.25) (layer F.Cu) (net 4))
 (segment (start 128.2192 64.7192) (end 128.8288 64.1096) (width 0.25) (layer F.Cu) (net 4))
 (segment (start 128.8288 64.1096) (end 136.144 64.1096) (width 0.25) (layer F.Cu) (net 4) (status 800000))
 (segment (start 136.144 64.1096) (end 136.652 64.6176) (width 0.25) (layer F.Cu) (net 4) (status C00000))
 (segment (start 129.8448 65.3288) (end 132.6896 65.3288) (width 0.25) (layer B.Cu) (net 5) (status 400000))
 (segment (start 134.5184 67.1576) (end 136.652 67.1576) (width 0.25) (layer B.Cu) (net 5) (status 800000))
 (segment (start 132.6896 65.3288) (end 134.5184 67.1576) (width 0.25) (layer B.Cu) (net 5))
 (segment (start 129.8448 67.8688) (end 132.6388 67.8688) (width 0.25) (layer B.Cu) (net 6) (status 400000))
 (segment (start 134.4676 69.6976) (end 136.652 69.6976) (width 0.25) (layer B.Cu) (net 6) (status 800000))
 (segment (start 132.6388 67.8688) (end 134.4676 69.6976) (width 0.25) (layer B.Cu) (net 6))
 (segment (start 129.8448 75.4888) (end 132.9944 75.4888) (width 0.25) (layer F.Cu) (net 7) (status 400000))
 (segment (start 133.7056 74.7776) (end 136.652 74.7776) (width 0.25) (layer F.Cu) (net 7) (status 800000))
 (segment (start 132.9944 75.4888) (end 133.7056 74.7776) (width 0.25) (layer F.Cu) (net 7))
 (segment (start 129.8448 70.4088) (end 131.8768 70.4088) (width 0.25) (layer B.Cu) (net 8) (status 400000))
 (segment (start 133.8072 74.4728) (end 136.652 77.3176) (width 0.25) (layer B.Cu) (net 8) (status 800000))
 (segment (start 133.8072 72.3392) (end 133.8072 74.4728) (width 0.25) (layer B.Cu) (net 8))
 (segment (start 131.8768 70.4088) (end 133.8072 72.3392) (width 0.25) (layer B.Cu) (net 8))
 (segment (start 129.8448 80.5688) (end 135.9408 80.5688) (width 0.25) (layer B.Cu) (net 9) (status 400000))
 (segment (start 135.9408 80.5688) (end 136.652 79.8576) (width 0.25) (layer B.Cu) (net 9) (status 800000))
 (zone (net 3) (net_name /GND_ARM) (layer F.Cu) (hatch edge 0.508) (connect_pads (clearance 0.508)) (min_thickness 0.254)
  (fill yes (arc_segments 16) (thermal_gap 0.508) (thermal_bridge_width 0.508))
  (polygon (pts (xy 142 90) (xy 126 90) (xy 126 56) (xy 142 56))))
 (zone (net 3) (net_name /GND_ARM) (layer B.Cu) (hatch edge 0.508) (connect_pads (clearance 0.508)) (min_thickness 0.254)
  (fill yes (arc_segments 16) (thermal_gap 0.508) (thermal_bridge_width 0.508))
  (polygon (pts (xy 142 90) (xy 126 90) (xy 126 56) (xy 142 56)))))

